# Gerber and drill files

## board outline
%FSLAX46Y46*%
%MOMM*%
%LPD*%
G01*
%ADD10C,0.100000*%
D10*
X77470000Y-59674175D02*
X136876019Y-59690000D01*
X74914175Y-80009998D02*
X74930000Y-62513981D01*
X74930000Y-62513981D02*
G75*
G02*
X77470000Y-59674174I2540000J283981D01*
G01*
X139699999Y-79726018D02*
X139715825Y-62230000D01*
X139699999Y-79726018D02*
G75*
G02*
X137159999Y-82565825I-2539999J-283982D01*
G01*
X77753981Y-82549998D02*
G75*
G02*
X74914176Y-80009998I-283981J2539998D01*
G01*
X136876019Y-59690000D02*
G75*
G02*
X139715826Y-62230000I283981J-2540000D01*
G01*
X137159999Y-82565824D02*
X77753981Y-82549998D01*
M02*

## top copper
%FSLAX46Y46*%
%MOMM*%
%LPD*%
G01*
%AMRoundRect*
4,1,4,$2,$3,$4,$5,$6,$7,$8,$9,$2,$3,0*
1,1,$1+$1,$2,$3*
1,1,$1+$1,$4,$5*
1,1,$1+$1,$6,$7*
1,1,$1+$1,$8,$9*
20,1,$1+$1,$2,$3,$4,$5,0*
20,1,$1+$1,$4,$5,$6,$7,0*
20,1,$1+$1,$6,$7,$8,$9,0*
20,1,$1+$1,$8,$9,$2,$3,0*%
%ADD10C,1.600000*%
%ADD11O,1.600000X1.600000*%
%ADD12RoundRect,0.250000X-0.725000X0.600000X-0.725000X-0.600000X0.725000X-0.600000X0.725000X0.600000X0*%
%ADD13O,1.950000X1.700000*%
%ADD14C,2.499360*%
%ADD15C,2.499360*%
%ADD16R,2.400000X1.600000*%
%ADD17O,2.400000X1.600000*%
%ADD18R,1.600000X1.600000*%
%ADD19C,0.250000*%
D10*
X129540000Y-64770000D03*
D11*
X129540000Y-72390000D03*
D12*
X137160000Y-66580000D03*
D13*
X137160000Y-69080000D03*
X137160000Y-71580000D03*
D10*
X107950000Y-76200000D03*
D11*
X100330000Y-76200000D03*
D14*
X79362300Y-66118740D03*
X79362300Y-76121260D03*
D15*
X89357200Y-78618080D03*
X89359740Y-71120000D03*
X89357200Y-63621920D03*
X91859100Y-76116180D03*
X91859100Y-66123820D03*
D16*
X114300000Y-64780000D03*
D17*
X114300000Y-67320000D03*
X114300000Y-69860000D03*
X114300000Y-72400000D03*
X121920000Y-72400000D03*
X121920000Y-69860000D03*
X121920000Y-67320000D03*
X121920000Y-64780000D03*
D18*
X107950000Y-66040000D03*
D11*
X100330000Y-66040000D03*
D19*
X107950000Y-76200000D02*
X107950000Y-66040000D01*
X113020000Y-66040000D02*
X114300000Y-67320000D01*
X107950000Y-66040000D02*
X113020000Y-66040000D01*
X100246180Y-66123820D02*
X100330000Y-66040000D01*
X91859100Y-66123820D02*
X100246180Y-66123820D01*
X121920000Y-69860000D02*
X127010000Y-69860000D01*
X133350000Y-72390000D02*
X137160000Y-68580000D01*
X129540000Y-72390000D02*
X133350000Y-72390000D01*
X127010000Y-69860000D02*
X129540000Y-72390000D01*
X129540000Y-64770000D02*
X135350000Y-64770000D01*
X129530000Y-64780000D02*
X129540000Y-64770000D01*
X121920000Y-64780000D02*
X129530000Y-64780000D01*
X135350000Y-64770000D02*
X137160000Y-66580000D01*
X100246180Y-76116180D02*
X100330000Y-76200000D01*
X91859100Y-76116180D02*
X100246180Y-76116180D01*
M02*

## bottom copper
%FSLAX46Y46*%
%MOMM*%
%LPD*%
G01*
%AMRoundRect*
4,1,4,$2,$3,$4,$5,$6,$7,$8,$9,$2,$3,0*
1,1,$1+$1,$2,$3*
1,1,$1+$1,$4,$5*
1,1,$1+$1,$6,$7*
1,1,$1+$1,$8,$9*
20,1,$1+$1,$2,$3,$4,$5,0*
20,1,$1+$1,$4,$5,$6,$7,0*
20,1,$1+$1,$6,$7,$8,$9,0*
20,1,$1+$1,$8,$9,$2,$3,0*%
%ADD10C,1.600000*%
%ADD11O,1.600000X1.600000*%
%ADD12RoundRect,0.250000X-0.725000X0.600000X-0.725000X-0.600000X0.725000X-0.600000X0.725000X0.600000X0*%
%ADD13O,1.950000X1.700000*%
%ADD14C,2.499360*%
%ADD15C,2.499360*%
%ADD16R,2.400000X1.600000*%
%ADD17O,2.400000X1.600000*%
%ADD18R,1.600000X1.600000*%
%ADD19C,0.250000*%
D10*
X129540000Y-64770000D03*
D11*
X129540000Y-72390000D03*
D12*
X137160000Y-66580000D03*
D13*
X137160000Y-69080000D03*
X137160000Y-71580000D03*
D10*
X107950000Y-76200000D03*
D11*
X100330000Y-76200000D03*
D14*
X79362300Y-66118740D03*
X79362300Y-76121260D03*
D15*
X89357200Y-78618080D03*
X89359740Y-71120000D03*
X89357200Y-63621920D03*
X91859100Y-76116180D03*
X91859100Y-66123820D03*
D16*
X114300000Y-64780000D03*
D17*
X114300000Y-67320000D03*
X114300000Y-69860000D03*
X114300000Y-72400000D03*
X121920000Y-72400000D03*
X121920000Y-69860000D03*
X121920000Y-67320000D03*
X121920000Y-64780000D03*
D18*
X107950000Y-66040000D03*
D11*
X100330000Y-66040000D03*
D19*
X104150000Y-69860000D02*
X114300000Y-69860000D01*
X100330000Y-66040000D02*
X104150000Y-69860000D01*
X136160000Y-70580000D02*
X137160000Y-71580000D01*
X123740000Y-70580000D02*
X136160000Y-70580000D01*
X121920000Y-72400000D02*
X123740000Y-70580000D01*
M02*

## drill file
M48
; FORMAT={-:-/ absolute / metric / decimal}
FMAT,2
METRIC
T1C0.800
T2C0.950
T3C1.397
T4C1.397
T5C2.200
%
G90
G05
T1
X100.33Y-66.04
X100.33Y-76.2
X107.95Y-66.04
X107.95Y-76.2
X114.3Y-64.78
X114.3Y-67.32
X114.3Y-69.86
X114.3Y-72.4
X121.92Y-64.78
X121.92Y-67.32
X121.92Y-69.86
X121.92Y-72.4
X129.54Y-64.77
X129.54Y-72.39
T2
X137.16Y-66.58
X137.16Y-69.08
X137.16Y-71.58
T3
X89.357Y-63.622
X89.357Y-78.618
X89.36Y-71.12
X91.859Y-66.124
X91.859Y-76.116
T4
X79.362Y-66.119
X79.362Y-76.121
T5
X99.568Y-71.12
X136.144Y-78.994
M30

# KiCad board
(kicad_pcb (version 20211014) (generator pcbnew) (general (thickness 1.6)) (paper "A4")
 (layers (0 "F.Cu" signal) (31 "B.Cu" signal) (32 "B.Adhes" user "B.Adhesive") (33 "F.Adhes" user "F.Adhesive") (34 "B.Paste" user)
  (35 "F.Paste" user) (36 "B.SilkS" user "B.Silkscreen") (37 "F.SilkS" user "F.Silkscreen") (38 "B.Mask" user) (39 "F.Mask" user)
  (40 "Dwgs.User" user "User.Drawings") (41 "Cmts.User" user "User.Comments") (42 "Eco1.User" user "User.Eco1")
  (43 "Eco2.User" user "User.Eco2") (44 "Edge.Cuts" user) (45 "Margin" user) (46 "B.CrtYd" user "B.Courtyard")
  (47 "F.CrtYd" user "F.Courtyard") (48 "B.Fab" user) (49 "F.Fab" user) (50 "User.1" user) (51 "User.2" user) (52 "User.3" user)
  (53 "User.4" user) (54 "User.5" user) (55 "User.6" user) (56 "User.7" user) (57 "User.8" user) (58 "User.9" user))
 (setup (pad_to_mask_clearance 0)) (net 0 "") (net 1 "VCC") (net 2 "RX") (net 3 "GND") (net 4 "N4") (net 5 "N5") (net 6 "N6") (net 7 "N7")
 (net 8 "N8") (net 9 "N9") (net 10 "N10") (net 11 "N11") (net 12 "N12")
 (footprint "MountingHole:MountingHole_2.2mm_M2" (layer "F.Cu") (at 136.144 78.994)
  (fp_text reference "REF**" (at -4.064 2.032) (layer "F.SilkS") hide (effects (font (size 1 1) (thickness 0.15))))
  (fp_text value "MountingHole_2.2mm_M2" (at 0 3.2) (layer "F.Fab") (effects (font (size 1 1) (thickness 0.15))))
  (pad "" np_thru_hole circle (at 0 0) (size 2.2 2.2) (drill 2.2) (layers *.Cu *.Mask)))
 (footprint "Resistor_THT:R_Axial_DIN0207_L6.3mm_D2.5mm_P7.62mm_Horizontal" (layer "F.Cu") (at 129.54 64.77 -90)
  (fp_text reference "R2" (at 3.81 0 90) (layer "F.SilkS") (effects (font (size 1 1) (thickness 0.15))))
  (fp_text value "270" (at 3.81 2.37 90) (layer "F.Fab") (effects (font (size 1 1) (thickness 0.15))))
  (pad "1" thru_hole circle (at 0 0 270) (size 1.6 1.6) (drill 0.8) (layers *.Cu *.Mask) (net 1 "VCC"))
  (pad "2" thru_hole oval (at 7.62 0 270) (size 1.6 1.6) (drill 0.8) (layers *.Cu *.Mask) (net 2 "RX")))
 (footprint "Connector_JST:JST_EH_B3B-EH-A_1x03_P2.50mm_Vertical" (layer "F.Cu") (at 137.16 66.58 -90)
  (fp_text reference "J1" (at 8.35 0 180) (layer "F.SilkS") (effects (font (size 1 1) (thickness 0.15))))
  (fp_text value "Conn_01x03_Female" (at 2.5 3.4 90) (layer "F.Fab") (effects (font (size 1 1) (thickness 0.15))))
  (pad "1" thru_hole roundrect (at 0 0 270) (size 1.7 1.95) (drill 0.95) (layers *.Cu *.Mask) (roundrect_rratio 0.147059) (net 1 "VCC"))
  (pad "2" thru_hole oval (at 2.5 0 270) (size 1.7 1.95) (drill 0.95) (layers *.Cu *.Mask) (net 2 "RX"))
  (pad "3" thru_hole oval (at 5 0 270) (size 1.7 1.95) (drill 0.95) (layers *.Cu *.Mask) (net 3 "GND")))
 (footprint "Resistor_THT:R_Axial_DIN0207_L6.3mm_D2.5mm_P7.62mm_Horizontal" (layer "F.Cu") (at 107.95 76.2 180)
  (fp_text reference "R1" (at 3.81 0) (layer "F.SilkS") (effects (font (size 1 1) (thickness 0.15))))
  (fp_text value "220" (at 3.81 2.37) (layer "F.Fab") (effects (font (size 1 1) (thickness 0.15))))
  (pad "1" thru_hole circle (at 0 0 180) (size 1.6 1.6) (drill 0.8) (layers *.Cu *.Mask) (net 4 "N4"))
  (pad "2" thru_hole oval (at 7.62 0 180) (size 1.6 1.6) (drill 0.8) (layers *.Cu *.Mask) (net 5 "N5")))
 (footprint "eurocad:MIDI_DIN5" (layer "F.Cu") (at 86.36 71.12 -90)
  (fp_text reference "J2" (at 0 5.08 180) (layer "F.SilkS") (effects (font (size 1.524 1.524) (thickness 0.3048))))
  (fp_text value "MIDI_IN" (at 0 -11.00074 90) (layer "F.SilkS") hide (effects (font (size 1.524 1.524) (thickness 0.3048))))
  (pad "" np_thru_hole circle locked (at -5.00126 6.9977 270) (size 2.49936 2.49936) (drill 1.397) (layers *.Cu *.Mask "F.SilkS"))
  (pad "" np_thru_hole circle locked (at 5.00126 6.9977 270) (size 2.49936 2.49936) (drill 1.397) (layers *.Cu *.Mask "F.SilkS"))
  (pad "1" thru_hole circle locked (at 7.49808 -2.9972 270) (size 2.49936 2.49936) (drill 1.397) (layers *.Cu *.SilkS *.Mask) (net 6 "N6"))
  (pad "2" thru_hole circle locked (at 0 -2.99974 270) (size 2.49936 2.49936) (drill 1.397) (layers *.Cu *.SilkS *.Mask) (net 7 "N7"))
  (pad "3" thru_hole circle locked (at -7.49808 -2.9972 270) (size 2.49936 2.49936) (drill 1.397) (layers *.Cu *.SilkS *.Mask) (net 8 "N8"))
  (pad "4" thru_hole circle locked (at 4.99618 -5.4991 270) (size 2.49936 2.49936) (drill 1.397) (layers *.Cu *.SilkS *.Mask) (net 5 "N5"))
  (pad "5" thru_hole circle locked (at -4.99618 -5.4991 270) (size 2.49936 2.49936) (drill 1.397) (layers *.Cu *.SilkS *.Mask) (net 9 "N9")))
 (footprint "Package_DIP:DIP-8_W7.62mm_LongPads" (layer "F.Cu") (at 114.3 64.78)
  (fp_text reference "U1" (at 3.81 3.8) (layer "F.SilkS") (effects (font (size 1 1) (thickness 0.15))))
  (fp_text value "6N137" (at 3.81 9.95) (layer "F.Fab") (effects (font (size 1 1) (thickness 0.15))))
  (pad "1" thru_hole rect (at 0 0) (size 2.4 1.6) (drill 0.8) (layers *.Cu *.Mask) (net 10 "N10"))
  (pad "2" thru_hole oval (at 0 2.54) (size 2.4 1.6) (drill 0.8) (layers *.Cu *.Mask) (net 4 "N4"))
  (pad "3" thru_hole oval (at 0 5.08) (size 2.4 1.6) (drill 0.8) (layers *.Cu *.Mask) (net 9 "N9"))
  (pad "4" thru_hole oval (at 0 7.62) (size 2.4 1.6) (drill 0.8) (layers *.Cu *.Mask) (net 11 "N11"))
  (pad "5" thru_hole oval (at 7.62 7.62) (size 2.4 1.6) (drill 0.8) (layers *.Cu *.Mask) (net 3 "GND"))
  (pad "6" thru_hole oval (at 7.62 5.08) (size 2.4 1.6) (drill 0.8) (layers *.Cu *.Mask) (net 2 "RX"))
  (pad "7" thru_hole oval (at 7.62 2.54) (size 2.4 1.6) (drill 0.8) (layers *.Cu *.Mask) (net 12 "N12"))
  (pad "8" thru_hole oval (at 7.62 0) (size 2.4 1.6) (drill 0.8) (layers *.Cu *.Mask) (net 1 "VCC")))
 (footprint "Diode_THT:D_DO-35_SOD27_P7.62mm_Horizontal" (layer "F.Cu") (at 107.95 66.04 180)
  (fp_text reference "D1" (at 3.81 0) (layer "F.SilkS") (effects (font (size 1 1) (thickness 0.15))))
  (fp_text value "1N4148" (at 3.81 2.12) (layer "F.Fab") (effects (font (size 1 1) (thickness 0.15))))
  (pad "1" thru_hole rect (at 0 0 180) (size 1.6 1.6) (drill 0.8) (layers *.Cu *.Mask) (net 4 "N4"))
  (pad "2" thru_hole oval (at 7.62 0 180) (size 1.6 1.6) (drill 0.8) (layers *.Cu *.Mask) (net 9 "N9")))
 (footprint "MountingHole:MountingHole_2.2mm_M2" (layer "F.Cu") (at 99.568 71.12)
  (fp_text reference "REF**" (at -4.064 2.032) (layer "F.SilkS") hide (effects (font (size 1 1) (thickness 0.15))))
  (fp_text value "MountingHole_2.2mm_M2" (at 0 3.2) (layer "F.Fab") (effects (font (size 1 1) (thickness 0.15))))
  (pad "" np_thru_hole circle (at 0 0) (size 2.2 2.2) (drill 2.2) (layers *.Cu *.Mask)))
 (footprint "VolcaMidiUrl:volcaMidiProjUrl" (layer "B.Cu") (at 120.396 78.486 180)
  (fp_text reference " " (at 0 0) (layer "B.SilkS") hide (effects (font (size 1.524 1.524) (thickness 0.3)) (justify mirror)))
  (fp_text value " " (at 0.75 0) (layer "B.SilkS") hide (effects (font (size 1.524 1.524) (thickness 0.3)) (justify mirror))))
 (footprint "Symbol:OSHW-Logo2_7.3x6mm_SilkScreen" (layer "B.Cu") (at 113.284 78.486 180)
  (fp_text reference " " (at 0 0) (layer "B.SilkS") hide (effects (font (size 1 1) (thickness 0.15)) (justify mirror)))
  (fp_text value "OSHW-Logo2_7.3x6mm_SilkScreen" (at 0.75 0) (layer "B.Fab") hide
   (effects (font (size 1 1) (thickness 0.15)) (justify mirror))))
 (gr_line (start 77.47 59.674175) (end 136.876019 59.69) (layer "Edge.Cuts") (width 0.1))
 (gr_line (start 74.914175 80.009998) (end 74.93 62.513981) (layer "Edge.Cuts") (width 0.1))
 (gr_arc (start 74.93 62.513981) (mid 75.564999 60.526116) (end 77.47 59.674175) (layer "Edge.Cuts") (width 0.1))
 (gr_line (start 139.699999 79.726018) (end 139.715825 62.23) (layer "Edge.Cuts") (width 0.1))
 (gr_arc (start 139.699999 79.726018) (mid 139.065 81.713883) (end 137.159999 82.565824) (layer "Edge.Cuts") (width 0.1))
 (gr_arc (start 77.753981 82.549998) (mid 75.766116 81.914999) (end 74.914175 80.009998) (layer "Edge.Cuts") (width 0.1))
 (gr_arc (start 136.876019 59.69) (mid 138.863884 60.324999) (end 139.715825 62.23) (layer "Edge.Cuts") (width 0.1))
 (gr_line (start 137.159999 82.565824) (end 77.753981 82.549998) (layer "Edge.Cuts") (width 0.1))
 (segment (start 107.95 76.2) (end 107.95 66.04) (width 0.25) (layer "F.Cu") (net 4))
 (segment (start 113.02 66.04) (end 114.3 67.32) (width 0.25) (layer "F.Cu") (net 4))
 (segment (start 107.95 66.04) (end 113.02 66.04) (width 0.25) (layer "F.Cu") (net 4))
 (segment (start 100.24618 66.12382) (end 100.33 66.04) (width 0.25) (layer "F.Cu") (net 9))
 (segment (start 91.8591 66.12382) (end 100.24618 66.12382) (width 0.25) (layer "F.Cu") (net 9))
 (segment (start 104.15 69.86) (end 114.3 69.86) (width 0.25) (layer "B.Cu") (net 9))
 (segment (start 100.33 66.04) (end 104.15 69.86) (width 0.25) (layer "B.Cu") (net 9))
 (segment (start 121.92 69.86) (end 127.01 69.86) (width 0.25) (layer "F.Cu") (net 2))
 (segment (start 133.35 72.39) (end 137.16 68.58) (width 0.25) (layer "F.Cu") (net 2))
 (segment (start 129.54 72.39) (end 133.35 72.39) (width 0.25) (layer "F.Cu") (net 2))
 (segment (start 127.01 69.86) (end 129.54 72.39) (width 0.25) (layer "F.Cu") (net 2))
 (segment (start 129.54 64.77) (end 135.35 64.77) (width 0.25) (layer "F.Cu") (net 1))
 (segment (start 129.53 64.78) (end 129.54 64.77) (width 0.25) (layer "F.Cu") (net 1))
 (segment (start 121.92 64.78) (end 129.53 64.78) (width 0.25) (layer "F.Cu") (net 1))
 (segment (start 135.35 64.77) (end 137.16 66.58) (width 0.25) (layer "F.Cu") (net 1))
 (segment (start 136.16 70.58) (end 137.16 71.58) (width 0.25) (layer "B.Cu") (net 3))
 (segment (start 123.74 70.58) (end 136.16 70.58) (width 0.25) (layer "B.Cu") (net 3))
 (segment (start 121.92 72.4) (end 123.74 70.58) (width 0.25) (layer "B.Cu") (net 3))
 (segment (start 100.24618 76.11618) (end 100.33 76.2) (width 0.25) (layer "F.Cu") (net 5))
 (segment (start 91.8591 76.11618) (end 100.24618 76.11618) (width 0.25) (layer "F.Cu") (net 5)))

